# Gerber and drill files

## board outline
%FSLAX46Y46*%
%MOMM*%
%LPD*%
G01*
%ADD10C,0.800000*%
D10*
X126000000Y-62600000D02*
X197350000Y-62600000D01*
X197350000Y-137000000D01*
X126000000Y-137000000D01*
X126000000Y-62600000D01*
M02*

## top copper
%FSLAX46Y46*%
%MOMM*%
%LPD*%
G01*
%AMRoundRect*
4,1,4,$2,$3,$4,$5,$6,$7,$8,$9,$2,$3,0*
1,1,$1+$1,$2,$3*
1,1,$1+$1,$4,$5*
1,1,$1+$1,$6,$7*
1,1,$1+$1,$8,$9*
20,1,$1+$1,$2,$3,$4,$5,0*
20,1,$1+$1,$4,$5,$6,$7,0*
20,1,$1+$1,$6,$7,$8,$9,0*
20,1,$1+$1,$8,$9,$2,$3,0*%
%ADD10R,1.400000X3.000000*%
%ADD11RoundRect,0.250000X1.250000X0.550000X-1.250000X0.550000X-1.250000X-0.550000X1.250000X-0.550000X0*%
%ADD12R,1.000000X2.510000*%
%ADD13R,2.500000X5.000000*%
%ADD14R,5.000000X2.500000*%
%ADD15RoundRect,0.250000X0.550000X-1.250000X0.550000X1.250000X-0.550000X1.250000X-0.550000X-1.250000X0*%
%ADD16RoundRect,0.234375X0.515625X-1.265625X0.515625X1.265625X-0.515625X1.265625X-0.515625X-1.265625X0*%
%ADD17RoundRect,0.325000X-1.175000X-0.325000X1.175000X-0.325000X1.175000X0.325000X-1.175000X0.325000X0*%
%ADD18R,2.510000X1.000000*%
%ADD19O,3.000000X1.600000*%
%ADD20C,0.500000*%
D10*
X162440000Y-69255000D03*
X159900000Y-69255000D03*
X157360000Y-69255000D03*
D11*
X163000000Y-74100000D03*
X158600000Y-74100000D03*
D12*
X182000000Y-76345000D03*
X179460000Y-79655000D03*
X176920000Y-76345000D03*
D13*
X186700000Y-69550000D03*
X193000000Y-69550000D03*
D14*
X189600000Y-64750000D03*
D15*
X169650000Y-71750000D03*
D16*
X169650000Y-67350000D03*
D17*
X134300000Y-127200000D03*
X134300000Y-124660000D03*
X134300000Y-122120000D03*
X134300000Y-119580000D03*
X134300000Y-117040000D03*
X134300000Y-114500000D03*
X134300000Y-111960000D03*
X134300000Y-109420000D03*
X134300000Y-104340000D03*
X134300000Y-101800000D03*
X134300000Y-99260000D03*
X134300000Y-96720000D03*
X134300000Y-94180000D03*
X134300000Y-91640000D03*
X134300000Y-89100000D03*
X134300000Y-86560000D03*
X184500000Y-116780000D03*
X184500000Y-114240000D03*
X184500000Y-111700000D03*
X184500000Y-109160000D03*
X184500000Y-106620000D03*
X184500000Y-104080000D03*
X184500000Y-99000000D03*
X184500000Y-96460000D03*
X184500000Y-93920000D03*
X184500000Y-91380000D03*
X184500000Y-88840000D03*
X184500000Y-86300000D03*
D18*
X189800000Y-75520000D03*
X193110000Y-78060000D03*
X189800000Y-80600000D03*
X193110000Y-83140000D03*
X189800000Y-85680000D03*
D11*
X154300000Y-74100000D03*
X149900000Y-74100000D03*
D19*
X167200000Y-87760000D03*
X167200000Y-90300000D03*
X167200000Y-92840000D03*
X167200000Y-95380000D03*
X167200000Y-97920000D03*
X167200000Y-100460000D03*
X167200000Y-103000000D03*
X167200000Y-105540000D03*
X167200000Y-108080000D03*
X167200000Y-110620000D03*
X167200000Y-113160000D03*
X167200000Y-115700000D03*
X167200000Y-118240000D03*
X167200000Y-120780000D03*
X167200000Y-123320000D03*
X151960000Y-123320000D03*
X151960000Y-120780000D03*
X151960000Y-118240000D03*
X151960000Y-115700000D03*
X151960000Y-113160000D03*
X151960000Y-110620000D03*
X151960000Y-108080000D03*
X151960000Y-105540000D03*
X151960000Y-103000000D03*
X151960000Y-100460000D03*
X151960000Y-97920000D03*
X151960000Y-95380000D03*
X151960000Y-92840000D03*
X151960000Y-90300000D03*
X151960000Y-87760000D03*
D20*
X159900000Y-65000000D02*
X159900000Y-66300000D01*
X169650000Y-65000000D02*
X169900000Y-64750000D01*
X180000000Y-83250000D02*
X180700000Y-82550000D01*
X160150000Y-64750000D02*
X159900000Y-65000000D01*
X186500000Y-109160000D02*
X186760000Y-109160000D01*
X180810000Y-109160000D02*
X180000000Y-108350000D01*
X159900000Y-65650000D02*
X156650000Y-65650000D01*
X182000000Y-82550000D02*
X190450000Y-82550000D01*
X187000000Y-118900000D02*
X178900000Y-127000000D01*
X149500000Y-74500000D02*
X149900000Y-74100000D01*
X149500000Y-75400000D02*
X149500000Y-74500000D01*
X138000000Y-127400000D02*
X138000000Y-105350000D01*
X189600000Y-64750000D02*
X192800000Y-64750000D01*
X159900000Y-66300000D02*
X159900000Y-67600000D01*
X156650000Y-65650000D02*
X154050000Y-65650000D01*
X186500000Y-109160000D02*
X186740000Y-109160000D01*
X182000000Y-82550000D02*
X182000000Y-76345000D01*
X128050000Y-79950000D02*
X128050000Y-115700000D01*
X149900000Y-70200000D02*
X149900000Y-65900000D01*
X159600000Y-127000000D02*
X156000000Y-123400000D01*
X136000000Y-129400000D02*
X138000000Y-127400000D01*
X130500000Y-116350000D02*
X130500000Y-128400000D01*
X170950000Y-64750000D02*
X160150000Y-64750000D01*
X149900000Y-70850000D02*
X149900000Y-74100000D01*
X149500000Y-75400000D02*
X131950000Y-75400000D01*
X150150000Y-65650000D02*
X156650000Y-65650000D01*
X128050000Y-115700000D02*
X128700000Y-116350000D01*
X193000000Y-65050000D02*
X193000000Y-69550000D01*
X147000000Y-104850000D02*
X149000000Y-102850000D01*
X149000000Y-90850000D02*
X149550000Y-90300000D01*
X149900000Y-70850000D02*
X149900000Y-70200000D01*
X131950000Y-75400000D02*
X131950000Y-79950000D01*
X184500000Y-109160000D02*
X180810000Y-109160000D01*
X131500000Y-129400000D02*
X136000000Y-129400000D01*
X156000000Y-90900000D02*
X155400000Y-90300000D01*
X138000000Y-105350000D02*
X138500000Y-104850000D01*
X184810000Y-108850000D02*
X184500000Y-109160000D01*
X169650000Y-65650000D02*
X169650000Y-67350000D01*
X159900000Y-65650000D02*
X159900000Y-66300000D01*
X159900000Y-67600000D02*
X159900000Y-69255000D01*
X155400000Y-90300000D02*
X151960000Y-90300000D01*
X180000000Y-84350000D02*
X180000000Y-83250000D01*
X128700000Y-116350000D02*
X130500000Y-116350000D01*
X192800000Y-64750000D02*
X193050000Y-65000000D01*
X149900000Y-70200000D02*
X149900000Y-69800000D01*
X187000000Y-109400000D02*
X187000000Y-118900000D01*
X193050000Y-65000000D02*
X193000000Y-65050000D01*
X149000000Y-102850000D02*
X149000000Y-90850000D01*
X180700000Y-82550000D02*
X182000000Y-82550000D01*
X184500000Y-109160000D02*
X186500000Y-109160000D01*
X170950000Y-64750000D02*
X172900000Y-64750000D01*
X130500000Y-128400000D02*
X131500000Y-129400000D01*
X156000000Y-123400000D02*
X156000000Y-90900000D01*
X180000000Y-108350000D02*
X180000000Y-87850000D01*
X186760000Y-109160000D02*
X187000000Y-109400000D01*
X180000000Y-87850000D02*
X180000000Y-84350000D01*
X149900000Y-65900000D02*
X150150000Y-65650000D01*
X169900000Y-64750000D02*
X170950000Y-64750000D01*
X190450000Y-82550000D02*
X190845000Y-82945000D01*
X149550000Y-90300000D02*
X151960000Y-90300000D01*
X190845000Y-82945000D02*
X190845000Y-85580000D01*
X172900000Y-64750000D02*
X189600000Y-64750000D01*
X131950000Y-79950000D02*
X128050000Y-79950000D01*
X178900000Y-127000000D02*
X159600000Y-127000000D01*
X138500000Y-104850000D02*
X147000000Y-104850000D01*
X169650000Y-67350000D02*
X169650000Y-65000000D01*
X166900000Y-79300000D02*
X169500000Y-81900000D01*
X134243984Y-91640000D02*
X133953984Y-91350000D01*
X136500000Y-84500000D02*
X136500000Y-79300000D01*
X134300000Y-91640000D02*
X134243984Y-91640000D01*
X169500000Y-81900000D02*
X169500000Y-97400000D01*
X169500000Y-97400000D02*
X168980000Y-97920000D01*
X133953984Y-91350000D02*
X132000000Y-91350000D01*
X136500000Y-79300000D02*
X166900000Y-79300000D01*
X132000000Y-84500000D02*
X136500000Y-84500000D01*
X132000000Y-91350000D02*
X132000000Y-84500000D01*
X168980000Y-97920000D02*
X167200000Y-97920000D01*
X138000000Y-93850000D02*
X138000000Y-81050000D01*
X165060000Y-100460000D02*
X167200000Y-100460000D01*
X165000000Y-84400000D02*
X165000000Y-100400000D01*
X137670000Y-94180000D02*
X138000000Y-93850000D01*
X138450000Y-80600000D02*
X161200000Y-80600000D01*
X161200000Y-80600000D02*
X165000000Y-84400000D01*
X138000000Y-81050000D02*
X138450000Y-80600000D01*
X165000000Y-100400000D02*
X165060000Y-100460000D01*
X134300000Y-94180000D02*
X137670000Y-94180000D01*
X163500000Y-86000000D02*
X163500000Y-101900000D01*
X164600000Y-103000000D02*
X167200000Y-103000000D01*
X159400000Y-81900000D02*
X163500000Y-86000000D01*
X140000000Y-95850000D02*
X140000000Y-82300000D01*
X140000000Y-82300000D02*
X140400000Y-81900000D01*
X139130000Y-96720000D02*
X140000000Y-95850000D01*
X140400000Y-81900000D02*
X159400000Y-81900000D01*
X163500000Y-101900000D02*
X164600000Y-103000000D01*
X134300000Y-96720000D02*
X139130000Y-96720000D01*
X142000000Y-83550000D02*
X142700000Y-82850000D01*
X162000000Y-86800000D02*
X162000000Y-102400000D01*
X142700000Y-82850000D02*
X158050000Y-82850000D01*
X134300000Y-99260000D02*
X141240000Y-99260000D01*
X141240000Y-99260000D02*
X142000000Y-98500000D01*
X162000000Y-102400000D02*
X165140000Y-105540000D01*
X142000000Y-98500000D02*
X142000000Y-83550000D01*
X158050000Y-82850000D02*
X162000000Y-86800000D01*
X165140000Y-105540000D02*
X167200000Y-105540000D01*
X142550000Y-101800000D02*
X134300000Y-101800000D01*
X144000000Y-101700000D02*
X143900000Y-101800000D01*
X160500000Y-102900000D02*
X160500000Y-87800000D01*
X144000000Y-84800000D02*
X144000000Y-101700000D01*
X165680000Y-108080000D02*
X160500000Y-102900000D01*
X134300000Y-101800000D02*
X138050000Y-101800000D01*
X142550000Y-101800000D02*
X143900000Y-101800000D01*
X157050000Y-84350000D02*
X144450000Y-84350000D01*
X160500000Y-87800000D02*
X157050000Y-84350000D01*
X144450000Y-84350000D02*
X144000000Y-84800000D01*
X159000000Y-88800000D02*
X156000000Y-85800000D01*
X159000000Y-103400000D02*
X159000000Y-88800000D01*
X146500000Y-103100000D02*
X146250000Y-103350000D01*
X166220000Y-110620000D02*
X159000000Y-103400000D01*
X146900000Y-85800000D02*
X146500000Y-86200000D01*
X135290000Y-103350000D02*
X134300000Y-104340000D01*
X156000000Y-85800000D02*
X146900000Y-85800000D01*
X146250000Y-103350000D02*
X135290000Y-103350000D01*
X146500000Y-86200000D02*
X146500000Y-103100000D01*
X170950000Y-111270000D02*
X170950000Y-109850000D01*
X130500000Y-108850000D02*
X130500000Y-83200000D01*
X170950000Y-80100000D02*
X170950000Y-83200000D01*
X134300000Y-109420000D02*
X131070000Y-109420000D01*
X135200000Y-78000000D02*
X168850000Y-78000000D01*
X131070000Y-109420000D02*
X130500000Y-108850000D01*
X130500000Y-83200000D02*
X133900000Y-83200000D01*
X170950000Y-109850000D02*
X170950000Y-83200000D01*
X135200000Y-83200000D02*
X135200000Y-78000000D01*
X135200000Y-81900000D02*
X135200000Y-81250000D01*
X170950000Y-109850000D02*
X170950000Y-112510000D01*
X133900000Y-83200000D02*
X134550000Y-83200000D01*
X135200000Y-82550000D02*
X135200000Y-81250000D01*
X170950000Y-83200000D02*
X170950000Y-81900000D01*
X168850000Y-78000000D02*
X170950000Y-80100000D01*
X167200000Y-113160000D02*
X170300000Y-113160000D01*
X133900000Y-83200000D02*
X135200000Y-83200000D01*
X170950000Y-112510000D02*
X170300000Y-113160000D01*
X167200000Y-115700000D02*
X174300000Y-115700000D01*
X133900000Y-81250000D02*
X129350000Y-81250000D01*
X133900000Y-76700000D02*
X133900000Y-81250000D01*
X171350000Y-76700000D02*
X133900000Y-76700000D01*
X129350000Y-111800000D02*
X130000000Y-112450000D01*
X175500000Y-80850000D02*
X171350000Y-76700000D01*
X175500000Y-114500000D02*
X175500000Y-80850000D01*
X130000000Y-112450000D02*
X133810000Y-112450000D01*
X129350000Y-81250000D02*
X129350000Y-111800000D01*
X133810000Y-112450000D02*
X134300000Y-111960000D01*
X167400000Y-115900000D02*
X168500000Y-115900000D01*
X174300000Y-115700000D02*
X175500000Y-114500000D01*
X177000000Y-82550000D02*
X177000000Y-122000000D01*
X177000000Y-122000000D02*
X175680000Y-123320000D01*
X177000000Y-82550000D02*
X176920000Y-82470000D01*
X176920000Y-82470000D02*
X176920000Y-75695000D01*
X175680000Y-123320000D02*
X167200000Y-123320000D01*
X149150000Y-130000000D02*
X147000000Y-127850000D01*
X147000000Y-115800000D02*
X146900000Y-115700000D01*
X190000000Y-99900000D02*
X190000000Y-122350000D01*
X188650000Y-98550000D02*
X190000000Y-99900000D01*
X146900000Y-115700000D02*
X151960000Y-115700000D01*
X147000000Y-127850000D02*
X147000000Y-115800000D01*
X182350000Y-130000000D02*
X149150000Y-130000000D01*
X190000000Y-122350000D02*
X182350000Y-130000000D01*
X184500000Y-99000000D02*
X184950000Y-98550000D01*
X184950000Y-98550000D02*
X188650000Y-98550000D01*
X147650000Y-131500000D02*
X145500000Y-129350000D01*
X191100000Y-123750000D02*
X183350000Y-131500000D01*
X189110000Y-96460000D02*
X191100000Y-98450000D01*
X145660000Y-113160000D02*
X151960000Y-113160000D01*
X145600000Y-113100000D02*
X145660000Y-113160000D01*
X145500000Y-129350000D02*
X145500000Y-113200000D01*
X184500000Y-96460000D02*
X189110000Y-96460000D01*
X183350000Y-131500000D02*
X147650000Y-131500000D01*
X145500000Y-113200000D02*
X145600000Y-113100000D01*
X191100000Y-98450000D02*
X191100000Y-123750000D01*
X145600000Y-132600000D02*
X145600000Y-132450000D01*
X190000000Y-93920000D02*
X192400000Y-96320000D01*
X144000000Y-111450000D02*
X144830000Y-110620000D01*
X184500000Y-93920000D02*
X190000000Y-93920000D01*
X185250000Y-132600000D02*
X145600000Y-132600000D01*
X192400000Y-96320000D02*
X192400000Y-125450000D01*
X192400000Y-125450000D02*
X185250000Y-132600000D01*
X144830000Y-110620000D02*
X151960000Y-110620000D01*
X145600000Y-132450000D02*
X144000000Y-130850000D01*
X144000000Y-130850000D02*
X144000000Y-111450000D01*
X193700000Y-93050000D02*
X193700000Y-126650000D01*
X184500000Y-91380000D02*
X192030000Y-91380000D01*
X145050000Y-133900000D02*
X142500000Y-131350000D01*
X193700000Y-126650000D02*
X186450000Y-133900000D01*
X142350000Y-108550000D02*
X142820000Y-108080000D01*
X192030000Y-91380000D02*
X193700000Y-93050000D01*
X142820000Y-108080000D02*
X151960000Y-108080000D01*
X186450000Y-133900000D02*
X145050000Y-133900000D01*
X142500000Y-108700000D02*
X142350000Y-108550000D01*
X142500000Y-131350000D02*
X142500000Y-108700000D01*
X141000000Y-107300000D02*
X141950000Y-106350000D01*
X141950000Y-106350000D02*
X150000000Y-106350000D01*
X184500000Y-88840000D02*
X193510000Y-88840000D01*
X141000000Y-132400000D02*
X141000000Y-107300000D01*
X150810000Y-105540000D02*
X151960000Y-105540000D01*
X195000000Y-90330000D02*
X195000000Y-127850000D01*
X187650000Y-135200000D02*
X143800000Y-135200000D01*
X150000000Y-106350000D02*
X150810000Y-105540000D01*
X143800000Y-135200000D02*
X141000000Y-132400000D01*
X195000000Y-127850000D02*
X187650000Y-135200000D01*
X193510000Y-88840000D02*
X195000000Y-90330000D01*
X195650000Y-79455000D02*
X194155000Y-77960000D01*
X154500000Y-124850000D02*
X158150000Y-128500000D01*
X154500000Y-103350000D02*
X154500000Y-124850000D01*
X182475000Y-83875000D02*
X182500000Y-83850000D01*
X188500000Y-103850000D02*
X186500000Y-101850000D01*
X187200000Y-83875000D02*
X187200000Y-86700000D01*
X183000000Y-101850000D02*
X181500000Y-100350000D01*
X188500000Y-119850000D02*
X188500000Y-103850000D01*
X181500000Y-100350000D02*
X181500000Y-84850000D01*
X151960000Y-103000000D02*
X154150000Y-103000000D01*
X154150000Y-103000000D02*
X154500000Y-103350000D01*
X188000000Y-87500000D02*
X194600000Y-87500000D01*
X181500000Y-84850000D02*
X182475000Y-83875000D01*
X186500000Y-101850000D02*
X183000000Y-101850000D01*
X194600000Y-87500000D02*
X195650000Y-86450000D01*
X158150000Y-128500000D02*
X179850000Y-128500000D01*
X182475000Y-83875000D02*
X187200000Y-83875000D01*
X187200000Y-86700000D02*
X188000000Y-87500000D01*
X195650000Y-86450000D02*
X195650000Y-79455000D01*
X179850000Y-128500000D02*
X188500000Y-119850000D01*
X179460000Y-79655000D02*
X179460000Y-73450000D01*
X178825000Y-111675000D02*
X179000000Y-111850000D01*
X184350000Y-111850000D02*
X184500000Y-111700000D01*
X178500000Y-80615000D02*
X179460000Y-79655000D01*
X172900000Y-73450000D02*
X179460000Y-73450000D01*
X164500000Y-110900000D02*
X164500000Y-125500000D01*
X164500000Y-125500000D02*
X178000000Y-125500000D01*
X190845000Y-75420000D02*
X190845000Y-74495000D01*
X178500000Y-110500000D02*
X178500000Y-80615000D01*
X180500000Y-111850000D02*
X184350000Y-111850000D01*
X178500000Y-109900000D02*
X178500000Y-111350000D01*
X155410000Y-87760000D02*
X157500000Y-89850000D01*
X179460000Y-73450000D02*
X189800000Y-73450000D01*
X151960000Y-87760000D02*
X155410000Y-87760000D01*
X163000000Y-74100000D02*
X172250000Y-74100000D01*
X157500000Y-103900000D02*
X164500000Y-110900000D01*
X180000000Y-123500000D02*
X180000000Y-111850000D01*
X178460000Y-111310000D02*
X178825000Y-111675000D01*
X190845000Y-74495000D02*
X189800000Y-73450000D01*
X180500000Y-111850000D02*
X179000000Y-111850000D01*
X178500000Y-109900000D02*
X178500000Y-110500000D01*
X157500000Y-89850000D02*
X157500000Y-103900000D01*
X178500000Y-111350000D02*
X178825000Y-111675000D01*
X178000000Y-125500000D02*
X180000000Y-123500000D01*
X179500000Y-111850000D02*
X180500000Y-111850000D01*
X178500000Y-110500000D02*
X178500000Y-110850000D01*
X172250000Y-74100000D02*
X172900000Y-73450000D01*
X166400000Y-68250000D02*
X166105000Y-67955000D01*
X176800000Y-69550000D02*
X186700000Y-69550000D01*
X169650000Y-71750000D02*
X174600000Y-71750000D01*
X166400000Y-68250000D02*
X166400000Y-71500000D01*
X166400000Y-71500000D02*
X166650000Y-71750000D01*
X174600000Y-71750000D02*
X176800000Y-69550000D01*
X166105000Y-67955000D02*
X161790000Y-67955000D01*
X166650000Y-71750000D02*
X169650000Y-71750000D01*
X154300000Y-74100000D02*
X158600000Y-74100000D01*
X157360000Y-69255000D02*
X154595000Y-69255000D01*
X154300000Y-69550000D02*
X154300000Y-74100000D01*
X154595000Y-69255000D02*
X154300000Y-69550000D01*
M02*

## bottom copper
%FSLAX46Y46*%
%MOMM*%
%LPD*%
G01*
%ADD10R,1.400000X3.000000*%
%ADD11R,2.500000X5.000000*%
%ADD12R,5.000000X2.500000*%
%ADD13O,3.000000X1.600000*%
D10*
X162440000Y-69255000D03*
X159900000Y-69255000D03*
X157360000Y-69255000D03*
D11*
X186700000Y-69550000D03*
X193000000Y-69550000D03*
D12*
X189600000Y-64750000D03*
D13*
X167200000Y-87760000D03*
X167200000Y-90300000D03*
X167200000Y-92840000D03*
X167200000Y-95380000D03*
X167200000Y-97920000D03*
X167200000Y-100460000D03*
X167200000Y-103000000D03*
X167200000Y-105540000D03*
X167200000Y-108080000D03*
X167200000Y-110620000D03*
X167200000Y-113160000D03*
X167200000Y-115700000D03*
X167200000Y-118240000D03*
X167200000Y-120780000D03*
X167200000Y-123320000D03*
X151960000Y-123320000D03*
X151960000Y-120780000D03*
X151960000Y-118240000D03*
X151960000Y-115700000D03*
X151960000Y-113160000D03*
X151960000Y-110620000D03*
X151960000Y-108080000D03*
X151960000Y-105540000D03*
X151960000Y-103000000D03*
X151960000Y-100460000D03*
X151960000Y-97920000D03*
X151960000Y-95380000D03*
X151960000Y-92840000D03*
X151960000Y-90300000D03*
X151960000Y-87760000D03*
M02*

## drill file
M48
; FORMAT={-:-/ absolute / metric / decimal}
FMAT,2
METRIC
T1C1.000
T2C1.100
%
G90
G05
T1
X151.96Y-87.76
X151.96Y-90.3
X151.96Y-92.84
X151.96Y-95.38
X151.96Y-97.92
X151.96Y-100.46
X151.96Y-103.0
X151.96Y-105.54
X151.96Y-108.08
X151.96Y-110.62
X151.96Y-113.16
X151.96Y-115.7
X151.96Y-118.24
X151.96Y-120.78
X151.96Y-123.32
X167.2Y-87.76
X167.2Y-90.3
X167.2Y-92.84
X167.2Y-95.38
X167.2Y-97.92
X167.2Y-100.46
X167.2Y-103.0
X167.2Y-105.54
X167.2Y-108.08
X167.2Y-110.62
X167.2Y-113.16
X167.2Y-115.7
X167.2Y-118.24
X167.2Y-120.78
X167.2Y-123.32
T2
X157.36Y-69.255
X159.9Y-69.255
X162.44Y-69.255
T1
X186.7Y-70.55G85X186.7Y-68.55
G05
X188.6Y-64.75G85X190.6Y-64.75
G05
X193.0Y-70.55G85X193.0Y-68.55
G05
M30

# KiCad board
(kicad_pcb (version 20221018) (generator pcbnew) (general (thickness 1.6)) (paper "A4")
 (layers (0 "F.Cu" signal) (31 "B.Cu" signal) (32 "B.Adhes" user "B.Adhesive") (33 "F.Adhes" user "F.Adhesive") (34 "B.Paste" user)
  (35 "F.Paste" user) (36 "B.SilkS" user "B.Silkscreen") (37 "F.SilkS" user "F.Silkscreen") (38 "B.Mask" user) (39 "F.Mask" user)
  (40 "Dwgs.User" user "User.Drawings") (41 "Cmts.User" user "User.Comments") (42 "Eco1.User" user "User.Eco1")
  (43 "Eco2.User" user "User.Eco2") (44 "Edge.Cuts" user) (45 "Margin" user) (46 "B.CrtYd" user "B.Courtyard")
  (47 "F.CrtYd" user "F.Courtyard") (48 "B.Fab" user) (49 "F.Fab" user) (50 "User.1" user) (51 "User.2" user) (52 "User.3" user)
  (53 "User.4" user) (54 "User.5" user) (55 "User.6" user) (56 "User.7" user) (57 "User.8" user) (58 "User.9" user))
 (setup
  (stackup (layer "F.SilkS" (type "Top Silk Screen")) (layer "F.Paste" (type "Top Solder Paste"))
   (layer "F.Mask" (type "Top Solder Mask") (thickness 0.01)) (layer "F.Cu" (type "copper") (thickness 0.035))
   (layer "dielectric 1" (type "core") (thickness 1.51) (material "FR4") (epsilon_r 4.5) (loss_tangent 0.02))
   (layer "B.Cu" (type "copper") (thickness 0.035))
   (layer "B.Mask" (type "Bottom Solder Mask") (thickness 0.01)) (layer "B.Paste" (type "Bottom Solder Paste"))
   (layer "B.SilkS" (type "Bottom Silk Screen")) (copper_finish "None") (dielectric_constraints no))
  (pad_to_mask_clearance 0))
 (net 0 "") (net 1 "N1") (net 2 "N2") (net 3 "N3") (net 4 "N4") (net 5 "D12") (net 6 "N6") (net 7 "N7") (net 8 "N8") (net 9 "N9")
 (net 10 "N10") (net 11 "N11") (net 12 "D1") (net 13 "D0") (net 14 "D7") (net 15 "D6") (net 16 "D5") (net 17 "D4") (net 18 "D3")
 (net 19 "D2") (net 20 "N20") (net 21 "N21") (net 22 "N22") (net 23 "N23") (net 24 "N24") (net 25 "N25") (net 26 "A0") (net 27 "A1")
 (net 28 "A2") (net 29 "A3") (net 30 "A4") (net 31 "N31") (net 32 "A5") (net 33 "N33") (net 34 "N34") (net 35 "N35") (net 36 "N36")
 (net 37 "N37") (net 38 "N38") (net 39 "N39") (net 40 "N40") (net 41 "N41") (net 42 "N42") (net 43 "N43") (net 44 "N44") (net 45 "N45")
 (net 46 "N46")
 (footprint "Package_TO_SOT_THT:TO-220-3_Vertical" (layer "F.Cu") (at 162.44 69.255 180)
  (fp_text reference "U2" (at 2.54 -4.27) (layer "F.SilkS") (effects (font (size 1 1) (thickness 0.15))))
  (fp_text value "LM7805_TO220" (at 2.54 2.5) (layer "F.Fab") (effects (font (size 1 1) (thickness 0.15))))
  (pad "1" thru_hole rect (at 0 0 180) (size 1.4 3) (drill 1.1) (layers "*.Cu" "*.Mask") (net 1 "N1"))
  (pad "2" thru_hole rect (at 2.54 0 180) (size 1.4 3) (drill 1.1) (layers "*.Cu" "*.Mask") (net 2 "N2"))
  (pad "3" thru_hole rect (at 5.08 0 180) (size 1.4 3) (drill 1.1) (layers "*.Cu" "*.Mask") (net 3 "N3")))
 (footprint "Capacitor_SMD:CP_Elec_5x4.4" (layer "F.Cu") (at 160.8 74.1 180)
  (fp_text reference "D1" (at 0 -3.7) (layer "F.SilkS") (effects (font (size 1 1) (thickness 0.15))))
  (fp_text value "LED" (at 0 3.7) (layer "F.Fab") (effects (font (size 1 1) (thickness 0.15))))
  (pad "1" smd roundrect (at -2.2 0 180) (size 3 1.6) (layers "F.Cu" "F.Paste" "F.Mask") (roundrect_rratio 0.15625) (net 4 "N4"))
  (pad "2" smd roundrect (at 2.2 0 180) (size 3 1.6) (layers "F.Cu" "F.Paste" "F.Mask") (roundrect_rratio 0.15625) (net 3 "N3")))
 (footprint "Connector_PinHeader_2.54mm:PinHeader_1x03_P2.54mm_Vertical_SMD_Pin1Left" (layer "F.Cu") (at 179.46 78 -90)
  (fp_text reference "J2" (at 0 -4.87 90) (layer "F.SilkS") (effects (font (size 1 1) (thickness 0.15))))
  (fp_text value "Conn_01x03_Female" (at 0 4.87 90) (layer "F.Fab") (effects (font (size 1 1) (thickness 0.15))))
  (pad "1" smd rect (at -1.655 -2.54 270) (size 2.51 1) (layers "F.Cu" "F.Paste" "F.Mask") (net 2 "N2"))
  (pad "2" smd rect (at 1.655 0 270) (size 2.51 1) (layers "F.Cu" "F.Paste" "F.Mask") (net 4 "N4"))
  (pad "3" smd rect (at -1.655 2.54 270) (size 2.51 1) (layers "F.Cu" "F.Paste" "F.Mask") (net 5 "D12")))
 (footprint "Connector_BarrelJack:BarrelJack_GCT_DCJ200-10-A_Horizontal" (layer "F.Cu") (at 186.7 69.55 90)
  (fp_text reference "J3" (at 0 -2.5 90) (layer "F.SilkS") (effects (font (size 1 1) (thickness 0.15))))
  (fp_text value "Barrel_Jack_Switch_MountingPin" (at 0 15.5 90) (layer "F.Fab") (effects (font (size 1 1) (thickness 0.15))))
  (pad "1" thru_hole rect (at 0 0 90) (size 5 2.5) (drill oval 3 1) (layers "*.Cu" "*.Mask") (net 1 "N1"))
  (pad "2" thru_hole rect (at 0 6.3 90) (size 5 2.5) (drill oval 3 1) (layers "*.Cu" "*.Mask") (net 2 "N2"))
  (pad "3" thru_hole rect (at 4.8 2.9 90) (size 2.5 5) (drill oval 1 3) (layers "*.Cu" "*.Mask") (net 2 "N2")))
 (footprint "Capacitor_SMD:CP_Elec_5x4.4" (layer "F.Cu") (at 169.65 69.55 90)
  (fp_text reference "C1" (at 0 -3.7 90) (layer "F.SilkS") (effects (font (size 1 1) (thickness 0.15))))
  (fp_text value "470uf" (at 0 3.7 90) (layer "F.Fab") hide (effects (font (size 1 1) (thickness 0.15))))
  (pad "1" smd roundrect (at -2.2 0 90) (size 3 1.6) (layers "F.Cu" "F.Paste" "F.Mask") (roundrect_rratio 0.15625) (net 1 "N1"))
  (pad "2" smd roundrect (at 2.2 0 90) (size 3 1.5) (layers "F.Cu" "F.Paste" "F.Mask") (roundrect_rratio 0.15625) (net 2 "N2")))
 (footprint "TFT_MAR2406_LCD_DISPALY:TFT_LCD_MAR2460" (layer "F.Cu") (at 134.3 127.2)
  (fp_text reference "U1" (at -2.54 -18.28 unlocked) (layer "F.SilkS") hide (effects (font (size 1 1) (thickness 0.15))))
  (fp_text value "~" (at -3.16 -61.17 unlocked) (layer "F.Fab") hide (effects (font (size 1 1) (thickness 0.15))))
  (pad "1" smd roundrect (at 0 0) (size 3 1.3) (layers "F.Cu" "F.Paste" "F.Mask") (roundrect_rratio 0.25) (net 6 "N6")
   (thermal_bridge_angle 45))
  (pad "2" smd roundrect (at 0 -2.54) (size 3 1.3) (layers "F.Cu" "F.Paste" "F.Mask") (roundrect_rratio 0.25) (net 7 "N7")
   (thermal_bridge_angle 45))
  (pad "3" smd roundrect (at 0 -5.08) (size 3 1.3) (layers "F.Cu" "F.Paste" "F.Mask") (roundrect_rratio 0.25) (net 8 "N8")
   (thermal_bridge_angle 45))
  (pad "4" smd roundrect (at 0 -7.62) (size 3 1.3) (layers "F.Cu" "F.Paste" "F.Mask") (roundrect_rratio 0.25) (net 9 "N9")
   (thermal_bridge_angle 45))
  (pad "5" smd roundrect (at 0 -10.16) (size 3 1.3) (layers "F.Cu" "F.Paste" "F.Mask") (roundrect_rratio 0.25) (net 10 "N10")
   (thermal_bridge_angle 45))
  (pad "6" smd roundrect (at 0 -12.7) (size 3 1.3) (layers "F.Cu" "F.Paste" "F.Mask") (roundrect_rratio 0.25) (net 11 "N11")
   (thermal_bridge_angle 45))
  (pad "7" smd roundrect (at 0 -15.24) (size 3 1.3) (layers "F.Cu" "F.Paste" "F.Mask") (roundrect_rratio 0.25) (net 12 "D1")
   (thermal_bridge_angle 45))
  (pad "8" smd roundrect (at 0 -17.78) (size 3 1.3) (layers "F.Cu" "F.Paste" "F.Mask") (roundrect_rratio 0.25) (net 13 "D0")
   (thermal_bridge_angle 45))
  (pad "9" smd roundrect (at 0 -22.86) (size 3 1.3) (layers "F.Cu" "F.Paste" "F.Mask") (roundrect_rratio 0.25) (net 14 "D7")
   (thermal_bridge_angle 45))
  (pad "10" smd roundrect (at 0 -25.4) (size 3 1.3) (layers "F.Cu" "F.Paste" "F.Mask") (roundrect_rratio 0.25) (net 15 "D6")
   (thermal_bridge_angle 45))
  (pad "11" smd roundrect (at 0 -27.94) (size 3 1.3) (layers "F.Cu" "F.Paste" "F.Mask") (roundrect_rratio 0.25) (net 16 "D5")
   (thermal_bridge_angle 45))
  (pad "12" smd roundrect (at 0 -30.48) (size 3 1.3) (layers "F.Cu" "F.Paste" "F.Mask") (roundrect_rratio 0.25) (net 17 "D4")
   (thermal_bridge_angle 45))
  (pad "13" smd roundrect (at 0 -33.02) (size 3 1.3) (layers "F.Cu" "F.Paste" "F.Mask") (roundrect_rratio 0.25) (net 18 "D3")
   (thermal_bridge_angle 45))
  (pad "14" smd roundrect (at 0 -35.56) (size 3 1.3) (layers "F.Cu" "F.Paste" "F.Mask") (roundrect_rratio 0.25) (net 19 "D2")
   (thermal_bridge_angle 45))
  (pad "15" smd roundrect (at 0 -38.1) (size 3 1.3) (layers "F.Cu" "F.Paste" "F.Mask") (roundrect_rratio 0.25) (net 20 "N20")
   (thermal_bridge_angle 45))
  (pad "16" smd roundrect (at 0 -40.64) (size 3 1.3) (layers "F.Cu" "F.Paste" "F.Mask") (roundrect_rratio 0.25) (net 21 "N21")
   (thermal_bridge_angle 45))
  (pad "17" smd roundrect (at 50.2 -10.42) (size 3 1.3) (layers "F.Cu" "F.Paste" "F.Mask") (roundrect_rratio 0.25) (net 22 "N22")
   (thermal_bridge_angle 45))
  (pad "18" smd roundrect (at 50.2 -12.96) (size 3 1.3) (layers "F.Cu" "F.Paste" "F.Mask") (roundrect_rratio 0.25) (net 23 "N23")
   (thermal_bridge_angle 45))
  (pad "19" smd roundrect (at 50.2 -15.5) (size 3 1.3) (layers "F.Cu" "F.Paste" "F.Mask") (roundrect_rratio 0.25) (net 4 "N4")
   (thermal_bridge_angle 45))
  (pad "20" smd roundrect (at 50.2 -18.04) (size 3 1.3) (layers "F.Cu" "F.Paste" "F.Mask") (roundrect_rratio 0.25) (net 2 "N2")
   (thermal_bridge_angle 45))
  (pad "21" smd roundrect (at 50.2 -20.58) (size 3 1.3) (layers "F.Cu" "F.Paste" "F.Mask") (roundrect_rratio 0.25) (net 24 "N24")
   (thermal_bridge_angle 45))
  (pad "22" smd roundrect (at 50.2 -23.12) (size 3 1.3) (layers "F.Cu" "F.Paste" "F.Mask") (roundrect_rratio 0.25) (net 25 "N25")
   (thermal_bridge_angle 45))
  (pad "23" smd roundrect (at 50.2 -28.2) (size 3 1.3) (layers "F.Cu" "F.Paste" "F.Mask") (roundrect_rratio 0.25) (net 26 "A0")
   (thermal_bridge_angle 45))
  (pad "24" smd roundrect (at 50.2 -30.74) (size 3 1.3) (layers "F.Cu" "F.Paste" "F.Mask") (roundrect_rratio 0.25) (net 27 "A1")
   (thermal_bridge_angle 45))
  (pad "25" smd roundrect (at 50.2 -33.28) (size 3 1.3) (layers "F.Cu" "F.Paste" "F.Mask") (roundrect_rratio 0.25) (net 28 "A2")
   (thermal_bridge_angle 45))
  (pad "26" smd roundrect (at 50.2 -35.82) (size 3 1.3) (layers "F.Cu" "F.Paste" "F.Mask") (roundrect_rratio 0.25) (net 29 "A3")
   (thermal_bridge_angle 45))
  (pad "27" smd roundrect (at 50.2 -38.36) (size 3 1.3) (layers "F.Cu" "F.Paste" "F.Mask") (roundrect_rratio 0.25) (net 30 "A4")
   (thermal_bridge_angle 45))
  (pad "28" smd roundrect (at 50.2 -40.9) (size 3 1.3) (layers "F.Cu" "F.Paste" "F.Mask") (roundrect_rratio 0.25) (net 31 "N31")
   (thermal_bridge_angle 45)))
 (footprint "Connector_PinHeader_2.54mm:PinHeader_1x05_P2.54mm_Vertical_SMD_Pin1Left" (layer "F.Cu") (at 191.455 80.6)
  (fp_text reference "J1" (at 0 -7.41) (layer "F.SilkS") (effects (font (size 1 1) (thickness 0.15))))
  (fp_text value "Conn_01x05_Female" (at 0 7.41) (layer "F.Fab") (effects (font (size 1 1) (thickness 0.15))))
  (pad "1" smd rect (at -1.655 -5.08) (size 2.51 1) (layers "F.Cu" "F.Paste" "F.Mask") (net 4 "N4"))
  (pad "2" smd rect (at 1.655 -2.54) (size 2.51 1) (layers "F.Cu" "F.Paste" "F.Mask") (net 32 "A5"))
  (pad "3" smd rect (at -1.655 0) (size 2.51 1) (layers "F.Cu" "F.Paste" "F.Mask") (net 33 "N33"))
  (pad "4" smd rect (at 1.655 2.54) (size 2.51 1) (layers "F.Cu" "F.Paste" "F.Mask") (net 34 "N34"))
  (pad "5" smd rect (at -1.655 5.08) (size 2.51 1) (layers "F.Cu" "F.Paste" "F.Mask") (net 2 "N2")))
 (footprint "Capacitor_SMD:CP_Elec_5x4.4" (layer "F.Cu") (at 152.1 74.1 180)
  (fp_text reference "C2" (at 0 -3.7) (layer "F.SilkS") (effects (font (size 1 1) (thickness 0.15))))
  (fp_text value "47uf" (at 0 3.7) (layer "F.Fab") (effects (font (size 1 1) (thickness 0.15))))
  (pad "1" smd roundrect (at -2.2 0 180) (size 3 1.6) (layers "F.Cu" "F.Paste" "F.Mask") (roundrect_rratio 0.15625) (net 3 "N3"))
  (pad "2" smd roundrect (at 2.2 0 180) (size 3 1.6) (layers "F.Cu" "F.Paste" "F.Mask") (roundrect_rratio 0.15625) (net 2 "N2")))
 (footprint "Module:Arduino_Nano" (layer "B.Cu") (at 167.2 87.76 180)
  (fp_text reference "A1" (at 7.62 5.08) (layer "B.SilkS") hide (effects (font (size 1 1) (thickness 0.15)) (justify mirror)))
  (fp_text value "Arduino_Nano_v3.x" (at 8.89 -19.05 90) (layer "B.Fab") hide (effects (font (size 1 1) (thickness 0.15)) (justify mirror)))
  (pad "1" thru_hole oval (at 0 0 180) (size 3 1.6) (drill 1) (layers "*.Cu" "*.Mask") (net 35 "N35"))
  (pad "2" thru_hole oval (at 0 -2.54 180) (size 3 1.6) (drill 1) (layers "*.Cu" "*.Mask") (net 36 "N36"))
  (pad "3" thru_hole oval (at 0 -5.08 180) (size 3 1.6) (drill 1) (layers "*.Cu" "*.Mask") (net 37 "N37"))
  (pad "4" thru_hole oval (at 0 -7.62 180) (size 3 1.6) (drill 1) (layers "*.Cu" "*.Mask") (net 2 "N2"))
  (pad "5" thru_hole oval (at 0 -10.16 180) (size 3 1.6) (drill 1) (layers "*.Cu" "*.Mask") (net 19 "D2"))
  (pad "6" thru_hole oval (at 0 -12.7 180) (size 3 1.6) (drill 1) (layers "*.Cu" "*.Mask") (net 18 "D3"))
  (pad "7" thru_hole oval (at 0 -15.24 180) (size 3 1.6) (drill 1) (layers "*.Cu" "*.Mask") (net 17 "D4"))
  (pad "8" thru_hole oval (at 0 -17.78 180) (size 3 1.6) (drill 1) (layers "*.Cu" "*.Mask") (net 16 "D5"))
  (pad "9" thru_hole oval (at 0 -20.32 180) (size 3 1.6) (drill 1) (layers "*.Cu" "*.Mask") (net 15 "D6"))
  (pad "10" thru_hole oval (at 0 -22.86 180) (size 3 1.6) (drill 1) (layers "*.Cu" "*.Mask") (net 14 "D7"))
  (pad "11" thru_hole oval (at 0 -25.4 180) (size 3 1.6) (drill 1) (layers "*.Cu" "*.Mask") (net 13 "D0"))
  (pad "12" thru_hole oval (at 0 -27.94 180) (size 3 1.6) (drill 1) (layers "*.Cu" "*.Mask") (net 12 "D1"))
  (pad "13" thru_hole oval (at 0 -30.48 180) (size 3 1.6) (drill 1) (layers "*.Cu" "*.Mask") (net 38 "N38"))
  (pad "14" thru_hole oval (at 0 -33.02 180) (size 3 1.6) (drill 1) (layers "*.Cu" "*.Mask") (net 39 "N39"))
  (pad "15" thru_hole oval (at 0 -35.56 180) (size 3 1.6) (drill 1) (layers "*.Cu" "*.Mask") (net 5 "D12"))
  (pad "16" thru_hole oval (at 15.24 -35.56 180) (size 3 1.6) (drill 1) (layers "*.Cu" "*.Mask") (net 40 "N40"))
  (pad "17" thru_hole oval (at 15.24 -33.02 180) (size 3 1.6) (drill 1) (layers "*.Cu" "*.Mask") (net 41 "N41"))
  (pad "18" thru_hole oval (at 15.24 -30.48 180) (size 3 1.6) (drill 1) (layers "*.Cu" "*.Mask") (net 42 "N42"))
  (pad "19" thru_hole oval (at 15.24 -27.94 180) (size 3 1.6) (drill 1) (layers "*.Cu" "*.Mask") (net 26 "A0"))
  (pad "20" thru_hole oval (at 15.24 -25.4 180) (size 3 1.6) (drill 1) (layers "*.Cu" "*.Mask") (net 27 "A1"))
  (pad "21" thru_hole oval (at 15.24 -22.86 180) (size 3 1.6) (drill 1) (layers "*.Cu" "*.Mask") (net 28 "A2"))
  (pad "22" thru_hole oval (at 15.24 -20.32 180) (size 3 1.6) (drill 1) (layers "*.Cu" "*.Mask") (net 29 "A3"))
  (pad "23" thru_hole oval (at 15.24 -17.78 180) (size 3 1.6) (drill 1) (layers "*.Cu" "*.Mask") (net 30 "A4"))
  (pad "24" thru_hole oval (at 15.24 -15.24 180) (size 3 1.6) (drill 1) (layers "*.Cu" "*.Mask") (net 32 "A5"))
  (pad "25" thru_hole oval (at 15.24 -12.7 180) (size 3 1.6) (drill 1) (layers "*.Cu" "*.Mask") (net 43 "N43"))
  (pad "26" thru_hole oval (at 15.24 -10.16 180) (size 3 1.6) (drill 1) (layers "*.Cu" "*.Mask") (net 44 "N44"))
  (pad "27" thru_hole oval (at 15.24 -7.62 180) (size 3 1.6) (drill 1) (layers "*.Cu" "*.Mask") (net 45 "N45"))
  (pad "28" thru_hole oval (at 15.24 -5.08 180) (size 3 1.6) (drill 1) (layers "*.Cu" "*.Mask") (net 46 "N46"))
  (pad "29" thru_hole oval (at 15.24 -2.54 180) (size 3 1.6) (drill 1) (layers "*.Cu" "*.Mask") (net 2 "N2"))
  (pad "30" thru_hole oval (at 15.24 0 180) (size 3 1.6) (drill 1) (layers "*.Cu" "*.Mask") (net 4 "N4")))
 (gr_rect (start 126 62.6) (end 197.35 137) (stroke (width 0.8) (type default)) (fill none) (layer "Edge.Cuts"))
 (segment (start 159.9 65) (end 159.9 66.3) (width 0.5) (layer "F.Cu") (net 2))
 (segment (start 169.65 65) (end 169.9 64.75) (width 0.5) (layer "F.Cu") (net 2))
 (segment (start 180 83.25) (end 180.7 82.55) (width 0.5) (layer "F.Cu") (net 2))
 (segment (start 160.15 64.75) (end 159.9 65) (width 0.5) (layer "F.Cu") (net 2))
 (segment (start 186.5 109.16) (end 186.76 109.16) (width 0.5) (layer "F.Cu") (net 2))
 (segment (start 180.81 109.16) (end 180 108.35) (width 0.5) (layer "F.Cu") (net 2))
 (segment (start 159.9 65.65) (end 156.65 65.65) (width 0.5) (layer "F.Cu") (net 2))
 (segment (start 182 82.55) (end 190.45 82.55) (width 0.5) (layer "F.Cu") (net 2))
 (segment (start 187 118.9) (end 178.9 127) (width 0.5) (layer "F.Cu") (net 2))
 (segment (start 149.5 74.5) (end 149.9 74.1) (width 0.5) (layer "F.Cu") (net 2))
 (segment (start 149.5 75.4) (end 149.5 74.5) (width 0.5) (layer "F.Cu") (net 2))
 (segment (start 138 127.4) (end 138 105.35) (width 0.5) (layer "F.Cu") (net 2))
 (segment (start 189.6 64.75) (end 192.8 64.75) (width 0.5) (layer "F.Cu") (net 2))
 (segment (start 159.9 66.3) (end 159.9 67.6) (width 0.5) (layer "F.Cu") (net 2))
 (segment (start 156.65 65.65) (end 154.05 65.65) (width 0.5) (layer "F.Cu") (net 2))
 (segment (start 186.5 109.16) (end 186.74 109.16) (width 0.5) (layer "F.Cu") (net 2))
 (segment (start 182 82.55) (end 182 76.345) (width 0.5) (layer "F.Cu") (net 2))
 (segment (start 128.05 79.95) (end 128.05 115.7) (width 0.5) (layer "F.Cu") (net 2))
 (segment (start 149.9 70.2) (end 149.9 65.9) (width 0.5) (layer "F.Cu") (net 2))
 (segment (start 159.6 127) (end 156 123.4) (width 0.5) (layer "F.Cu") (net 2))
 (segment (start 136 129.4) (end 138 127.4) (width 0.5) (layer "F.Cu") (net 2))
 (segment (start 130.5 116.35) (end 130.5 128.4) (width 0.5) (layer "F.Cu") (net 2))
 (segment (start 170.95 64.75) (end 160.15 64.75) (width 0.5) (layer "F.Cu") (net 2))
 (segment (start 149.9 70.85) (end 149.9 74.1) (width 0.5) (layer "F.Cu") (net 2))
 (segment (start 149.5 75.4) (end 131.95 75.4) (width 0.5) (layer "F.Cu") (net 2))
 (segment (start 150.15 65.65) (end 156.65 65.65) (width 0.5) (layer "F.Cu") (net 2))
 (segment (start 128.05 115.7) (end 128.7 116.35) (width 0.5) (layer "F.Cu") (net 2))
 (segment (start 193 65.05) (end 193 69.55) (width 0.5) (layer "F.Cu") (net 2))
 (segment (start 147 104.85) (end 149 102.85) (width 0.5) (layer "F.Cu") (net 2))
 (segment (start 149 90.85) (end 149.55 90.3) (width 0.5) (layer "F.Cu") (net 2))
 (segment (start 149.9 70.85) (end 149.9 70.2) (width 0.5) (layer "F.Cu") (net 2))
 (segment (start 131.95 75.4) (end 131.95 79.95) (width 0.5) (layer "F.Cu") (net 2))
 (segment (start 184.5 109.16) (end 180.81 109.16) (width 0.5) (layer "F.Cu") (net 2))
 (segment (start 131.5 129.4) (end 136 129.4) (width 0.5) (layer "F.Cu") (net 2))
 (segment (start 156 90.9) (end 155.4 90.3) (width 0.5) (layer "F.Cu") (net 2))
 (segment (start 138 105.35) (end 138.5 104.85) (width 0.5) (layer "F.Cu") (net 2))
 (segment (start 184.81 108.85) (end 184.5 109.16) (width 0.5) (layer "F.Cu") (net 2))
 (segment (start 169.65 65.65) (end 169.65 67.35) (width 0.5) (layer "F.Cu") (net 2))
 (segment (start 159.9 65.65) (end 159.9 66.3) (width 0.5) (layer "F.Cu") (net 2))
 (segment (start 159.9 67.6) (end 159.9 69.255) (width 0.5) (layer "F.Cu") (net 2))
 (segment (start 155.4 90.3) (end 151.96 90.3) (width 0.5) (layer "F.Cu") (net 2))
 (segment (start 180 84.35) (end 180 83.25) (width 0.5) (layer "F.Cu") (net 2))
 (segment (start 128.7 116.35) (end 130.5 116.35) (width 0.5) (layer "F.Cu") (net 2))
 (segment (start 192.8 64.75) (end 193.05 65) (width 0.5) (layer "F.Cu") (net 2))
 (segment (start 149.9 70.2) (end 149.9 69.8) (width 0.5) (layer "F.Cu") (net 2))
 (segment (start 187 109.4) (end 187 118.9) (width 0.5) (layer "F.Cu") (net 2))
 (segment (start 193.05 65) (end 193 65.05) (width 0.5) (layer "F.Cu") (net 2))
 (segment (start 149 102.85) (end 149 90.85) (width 0.5) (layer "F.Cu") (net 2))
 (segment (start 180.7 82.55) (end 182 82.55) (width 0.5) (layer "F.Cu") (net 2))
 (segment (start 184.5 109.16) (end 186.5 109.16) (width 0.5) (layer "F.Cu") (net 2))
 (segment (start 170.95 64.75) (end 172.9 64.75) (width 0.5) (layer "F.Cu") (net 2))
 (segment (start 130.5 128.4) (end 131.5 129.4) (width 0.5) (layer "F.Cu") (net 2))
 (segment (start 156 123.4) (end 156 90.9) (width 0.5) (layer "F.Cu") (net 2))
 (segment (start 180 108.35) (end 180 87.85) (width 0.5) (layer "F.Cu") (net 2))
 (segment (start 186.76 109.16) (end 187 109.4) (width 0.5) (layer "F.Cu") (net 2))
 (segment (start 180 87.85) (end 180 84.35) (width 0.5) (layer "F.Cu") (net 2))
 (segment (start 149.9 65.9) (end 150.15 65.65) (width 0.5) (layer "F.Cu") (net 2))
 (segment (start 169.9 64.75) (end 170.95 64.75) (width 0.5) (layer "F.Cu") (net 2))
 (segment (start 190.45 82.55) (end 190.845 82.945) (width 0.5) (layer "F.Cu") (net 2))
 (segment (start 149.55 90.3) (end 151.96 90.3) (width 0.5) (layer "F.Cu") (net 2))
 (segment (start 190.845 82.945) (end 190.845 85.58) (width 0.5) (layer "F.Cu") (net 2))
 (segment (start 172.9 64.75) (end 189.6 64.75) (width 0.5) (layer "F.Cu") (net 2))
 (segment (start 131.95 79.95) (end 128.05 79.95) (width 0.5) (layer "F.Cu") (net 2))
 (segment (start 178.9 127) (end 159.6 127) (width 0.5) (layer "F.Cu") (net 2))
 (segment (start 138.5 104.85) (end 147 104.85) (width 0.5) (layer "F.Cu") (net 2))
 (segment (start 169.65 67.35) (end 169.65 65) (width 0.5) (layer "F.Cu") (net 2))
 (segment (start 166.9 79.3) (end 169.5 81.9) (width 0.5) (layer "F.Cu") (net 19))
 (segment (start 134.243984 91.64) (end 133.953984 91.35) (width 0.5) (layer "F.Cu") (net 19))
 (segment (start 136.5 84.5) (end 136.5 79.3) (width 0.5) (layer "F.Cu") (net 19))
 (segment (start 134.3 91.64) (end 134.243984 91.64) (width 0.5) (layer "F.Cu") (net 19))
 (segment (start 169.5 81.9) (end 169.5 97.4) (width 0.5) (layer "F.Cu") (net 19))
 (segment (start 169.5 97.4) (end 168.98 97.92) (width 0.5) (layer "F.Cu") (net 19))
 (segment (start 133.953984 91.35) (end 132 91.35) (width 0.5) (layer "F.Cu") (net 19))
 (segment (start 136.5 79.3) (end 166.9 79.3) (width 0.5) (layer "F.Cu") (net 19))
 (segment (start 132 84.5) (end 136.5 84.5) (width 0.5) (layer "F.Cu") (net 19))
 (segment (start 132 91.35) (end 132 84.5) (width 0.5) (layer "F.Cu") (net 19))
 (segment (start 168.98 97.92) (end 167.2 97.92) (width 0.5) (layer "F.Cu") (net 19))
 (segment (start 138 93.85) (end 138 81.05) (width 0.5) (layer "F.Cu") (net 18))
 (segment (start 165.06 100.46) (end 167.2 100.46) (width 0.5) (layer "F.Cu") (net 18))
 (segment (start 165 84.4) (end 165 100.4) (width 0.5) (layer "F.Cu") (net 18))
 (segment (start 137.67 94.18) (end 138 93.85) (width 0.5) (layer "F.Cu") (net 18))
 (segment (start 138.45 80.6) (end 161.2 80.6) (width 0.5) (layer "F.Cu") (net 18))
 (segment (start 161.2 80.6) (end 165 84.4) (width 0.5) (layer "F.Cu") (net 18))
 (segment (start 138 81.05) (end 138.45 80.6) (width 0.5) (layer "F.Cu") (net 18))
 (segment (start 165 100.4) (end 165.06 100.46) (width 0.5) (layer "F.Cu") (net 18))
 (segment (start 134.3 94.18) (end 137.67 94.18) (width 0.5) (layer "F.Cu") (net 18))
 (segment (start 163.5 86) (end 163.5 101.9) (width 0.5) (layer "F.Cu") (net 17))
 (segment (start 164.6 103) (end 167.2 103) (width 0.5) (layer "F.Cu") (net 17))
 (segment (start 159.4 81.9) (end 163.5 86) (width 0.5) (layer "F.Cu") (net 17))
 (segment (start 140 95.85) (end 140 82.3) (width 0.5) (layer "F.Cu") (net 17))
 (segment (start 140 82.3) (end 140.4 81.9) (width 0.5) (layer "F.Cu") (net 17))
 (segment (start 139.13 96.72) (end 140 95.85) (width 0.5) (layer "F.Cu") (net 17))
 (segment (start 140.4 81.9) (end 159.4 81.9) (width 0.5) (layer "F.Cu") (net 17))
 (segment (start 163.5 101.9) (end 164.6 103) (width 0.5) (layer "F.Cu") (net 17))
 (segment (start 134.3 96.72) (end 139.13 96.72) (width 0.5) (layer "F.Cu") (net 17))
 (segment (start 142 83.55) (end 142.7 82.85) (width 0.5) (layer "F.Cu") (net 16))
 (segment (start 162 86.8) (end 162 102.4) (width 0.5) (layer "F.Cu") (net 16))
 (segment (start 142.7 82.85) (end 158.05 82.85) (width 0.5) (layer "F.Cu") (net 16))
 (segment (start 134.3 99.26) (end 141.24 99.26) (width 0.5) (layer "F.Cu") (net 16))
 (segment (start 141.24 99.26) (end 142 98.5) (width 0.5) (layer "F.Cu") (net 16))
 (segment (start 162 102.4) (end 165.14 105.54) (width 0.5) (layer "F.Cu") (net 16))
 (segment (start 142 98.5) (end 142 83.55) (width 0.5) (layer "F.Cu") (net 16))
 (segment (start 158.05 82.85) (end 162 86.8) (width 0.5) (layer "F.Cu") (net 16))
 (segment (start 165.14 105.54) (end 167.2 105.54) (width 0.5) (layer "F.Cu") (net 16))
 (segment (start 142.55 101.8) (end 134.3 101.8) (width 0.5) (layer "F.Cu") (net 15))
 (segment (start 144 101.7) (end 143.9 101.8) (width 0.5) (layer "F.Cu") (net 15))
 (segment (start 160.5 102.9) (end 160.5 87.8) (width 0.5) (layer "F.Cu") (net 15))
 (segment (start 144 84.8) (end 144 101.7) (width 0.5) (layer "F.Cu") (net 15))
 (segment (start 165.68 108.08) (end 160.5 102.9) (width 0.5) (layer "F.Cu") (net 15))
 (segment (start 134.3 101.8) (end 138.05 101.8) (width 0.5) (layer "F.Cu") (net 15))
 (segment (start 142.55 101.8) (end 143.9 101.8) (width 0.5) (layer "F.Cu") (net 15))
 (segment (start 157.05 84.35) (end 144.45 84.35) (width 0.5) (layer "F.Cu") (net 15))
 (segment (start 160.5 87.8) (end 157.05 84.35) (width 0.5) (layer "F.Cu") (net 15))
 (segment (start 144.45 84.35) (end 144 84.8) (width 0.5) (layer "F.Cu") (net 15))
 (segment (start 159 88.8) (end 156 85.8) (width 0.5) (layer "F.Cu") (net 14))
 (segment (start 159 103.4) (end 159 88.8) (width 0.5) (layer "F.Cu") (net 14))
 (segment (start 146.5 103.1) (end 146.25 103.35) (width 0.5) (layer "F.Cu") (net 14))
 (segment (start 166.22 110.62) (end 159 103.4) (width 0.5) (layer "F.Cu") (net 14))
 (segment (start 146.9 85.8) (end 146.5 86.2) (width 0.5) (layer "F.Cu") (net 14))
 (segment (start 135.29 103.35) (end 134.3 104.34) (width 0.5) (layer "F.Cu") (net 14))
 (segment (start 156 85.8) (end 146.9 85.8) (width 0.5) (layer "F.Cu") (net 14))
 (segment (start 146.25 103.35) (end 135.29 103.35) (width 0.5) (layer "F.Cu") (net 14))
 (segment (start 146.5 86.2) (end 146.5 103.1) (width 0.5) (layer "F.Cu") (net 14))
 (segment (start 170.95 111.27) (end 170.95 109.85) (width 0.5) (layer "F.Cu") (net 13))
 (segment (start 130.5 108.85) (end 130.5 83.2) (width 0.5) (layer "F.Cu") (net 13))
 (segment (start 170.95 80.1) (end 170.95 83.2) (width 0.5) (layer "F.Cu") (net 13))
 (segment (start 134.3 109.42) (end 131.07 109.42) (width 0.5) (layer "F.Cu") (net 13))
 (segment (start 135.2 78) (end 168.85 78) (width 0.5) (layer "F.Cu") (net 13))
 (segment (start 131.07 109.42) (end 130.5 108.85) (width 0.5) (layer "F.Cu") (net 13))
 (segment (start 130.5 83.2) (end 133.9 83.2) (width 0.5) (layer "F.Cu") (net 13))
 (segment (start 170.95 109.85) (end 170.95 83.2) (width 0.5) (layer "F.Cu") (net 13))
 (segment (start 135.2 83.2) (end 135.2 78) (width 0.5) (layer "F.Cu") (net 13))
 (segment (start 135.2 81.9) (end 135.2 81.25) (width 0.5) (layer "F.Cu") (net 13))
 (segment (start 170.95 109.85) (end 170.95 112.51) (width 0.5) (layer "F.Cu") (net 13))
 (segment (start 133.9 83.2) (end 134.55 83.2) (width 0.5) (layer "F.Cu") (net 13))
 (segment (start 135.2 82.55) (end 135.2 81.25) (width 0.5) (layer "F.Cu") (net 13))
 (segment (start 170.95 83.2) (end 170.95 81.9) (width 0.5) (layer "F.Cu") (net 13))
 (segment (start 168.85 78) (end 170.95 80.1) (width 0.5) (layer "F.Cu") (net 13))
 (segment (start 167.2 113.16) (end 170.3 113.16) (width 0.5) (layer "F.Cu") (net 13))
 (segment (start 133.9 83.2) (end 135.2 83.2) (width 0.5) (layer "F.Cu") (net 13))
 (segment (start 170.95 112.51) (end 170.3 113.16) (width 0.5) (layer "F.Cu") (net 13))
 (segment (start 167.2 115.7) (end 174.3 115.7) (width 0.5) (layer "F.Cu") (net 12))
 (segment (start 133.9 81.25) (end 129.35 81.25) (width 0.5) (layer "F.Cu") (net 12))
 (segment (start 133.9 76.7) (end 133.9 81.25) (width 0.5) (layer "F.Cu") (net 12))
 (segment (start 171.35 76.7) (end 133.9 76.7) (width 0.5) (layer "F.Cu") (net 12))
 (segment (start 129.35 111.8) (end 130 112.45) (width 0.5) (layer "F.Cu") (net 12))
 (segment (start 175.5 80.85) (end 171.35 76.7) (width 0.5) (layer "F.Cu") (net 12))
 (segment (start 175.5 114.5) (end 175.5 80.85) (width 0.5) (layer "F.Cu") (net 12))
 (segment (start 130 112.45) (end 133.81 112.45) (width 0.5) (layer "F.Cu") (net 12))
 (segment (start 129.35 81.25) (end 129.35 111.8) (width 0.5) (layer "F.Cu") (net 12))
 (segment (start 133.81 112.45) (end 134.3 111.96) (width 0.5) (layer "F.Cu") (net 12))
 (segment (start 167.4 115.9) (end 168.5 115.9) (width 0.5) (layer "F.Cu") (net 12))
 (segment (start 174.3 115.7) (end 175.5 114.5) (width 0.5) (layer "F.Cu") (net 12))
 (segment (start 177 82.55) (end 177 122) (width 0.5) (layer "F.Cu") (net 5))
 (segment (start 177 122) (end 175.68 123.32) (width 0.5) (layer "F.Cu") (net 5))
 (segment (start 177 82.55) (end 176.92 82.47) (width 0.5) (layer "F.Cu") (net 5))
 (segment (start 176.92 82.47) (end 176.92 75.695) (width 0.5) (layer "F.Cu") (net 5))
 (segment (start 175.68 123.32) (end 167.2 123.32) (width 0.5) (layer "F.Cu") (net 5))
 (segment (start 149.15 130) (end 147 127.85) (width 0.5) (layer "F.Cu") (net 26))
 (segment (start 147 115.8) (end 146.9 115.7) (width 0.5) (layer "F.Cu") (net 26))
 (segment (start 190 99.9) (end 190 122.35) (width 0.5) (layer "F.Cu") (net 26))
 (segment (start 188.65 98.55) (end 190 99.9) (width 0.5) (layer "F.Cu") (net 26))
 (segment (start 146.9 115.7) (end 151.96 115.7) (width 0.5) (layer "F.Cu") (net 26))
 (segment (start 147 127.85) (end 147 115.8) (width 0.5) (layer "F.Cu") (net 26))
 (segment (start 182.35 130) (end 149.15 130) (width 0.5) (layer "F.Cu") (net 26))
 (segment (start 190 122.35) (end 182.35 130) (width 0.5) (layer "F.Cu") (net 26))
 (segment (start 184.5 99) (end 184.95 98.55) (width 0.5) (layer "F.Cu") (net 26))
 (segment (start 184.95 98.55) (end 188.65 98.55) (width 0.5) (layer "F.Cu") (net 26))
 (segment (start 147.65 131.5) (end 145.5 129.35) (width 0.5) (layer "F.Cu") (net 27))
 (segment (start 191.1 123.75) (end 183.35 131.5) (width 0.5) (layer "F.Cu") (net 27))
 (segment (start 189.11 96.46) (end 191.1 98.45) (width 0.5) (layer "F.Cu") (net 27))
 (segment (start 145.66 113.16) (end 151.96 113.16) (width 0.5) (layer "F.Cu") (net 27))
 (segment (start 145.6 113.1) (end 145.66 113.16) (width 0.5) (layer "F.Cu") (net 27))
 (segment (start 145.5 129.35) (end 145.5 113.2) (width 0.5) (layer "F.Cu") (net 27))
 (segment (start 184.5 96.46) (end 189.11 96.46) (width 0.5) (layer "F.Cu") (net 27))
 (segment (start 183.35 131.5) (end 147.65 131.5) (width 0.5) (layer "F.Cu") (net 27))
 (segment (start 145.5 113.2) (end 145.6 113.1) (width 0.5) (layer "F.Cu") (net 27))
 (segment (start 191.1 98.45) (end 191.1 123.75) (width 0.5) (layer "F.Cu") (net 27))
 (segment (start 145.6 132.6) (end 145.6 132.45) (width 0.5) (layer "F.Cu") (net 28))
 (segment (start 190 93.92) (end 192.4 96.32) (width 0.5) (layer "F.Cu") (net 28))
 (segment (start 144 111.45) (end 144.83 110.62) (width 0.5) (layer "F.Cu") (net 28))
 (segment (start 184.5 93.92) (end 190 93.92) (width 0.5) (layer "F.Cu") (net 28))
 (segment (start 185.25 132.6) (end 145.6 132.6) (width 0.5) (layer "F.Cu") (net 28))
 (segment (start 192.4 96.32) (end 192.4 125.45) (width 0.5) (layer "F.Cu") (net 28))
 (segment (start 192.4 125.45) (end 185.25 132.6) (width 0.5) (layer "F.Cu") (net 28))
 (segment (start 144.83 110.62) (end 151.96 110.62) (width 0.5) (layer "F.Cu") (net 28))
 (segment (start 145.6 132.45) (end 144 130.85) (width 0.5) (layer "F.Cu") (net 28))
 (segment (start 144 130.85) (end 144 111.45) (width 0.5) (layer "F.Cu") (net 28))
 (segment (start 193.7 93.05) (end 193.7 126.65) (width 0.5) (layer "F.Cu") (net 29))
 (segment (start 184.5 91.38) (end 192.03 91.38) (width 0.5) (layer "F.Cu") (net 29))
 (segment (start 145.05 133.9) (end 142.5 131.35) (width 0.5) (layer "F.Cu") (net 29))
 (segment (start 193.7 126.65) (end 186.45 133.9) (width 0.5) (layer "F.Cu") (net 29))
 (segment (start 142.35 108.55) (end 142.82 108.08) (width 0.5) (layer "F.Cu") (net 29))
 (segment (start 192.03 91.38) (end 193.7 93.05) (width 0.5) (layer "F.Cu") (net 29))
 (segment (start 142.82 108.08) (end 151.96 108.08) (width 0.5) (layer "F.Cu") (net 29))
 (segment (start 186.45 133.9) (end 145.05 133.9) (width 0.5) (layer "F.Cu") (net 29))
 (segment (start 142.5 108.7) (end 142.35 108.55) (width 0.5) (layer "F.Cu") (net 29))
 (segment (start 142.5 131.35) (end 142.5 108.7) (width 0.5) (layer "F.Cu") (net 29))
 (segment (start 141 107.3) (end 141.95 106.35) (width 0.5) (layer "F.Cu") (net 30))
 (segment (start 141.95 106.35) (end 150 106.35) (width 0.5) (layer "F.Cu") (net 30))
 (segment (start 184.5 88.84) (end 193.51 88.84) (width 0.5) (layer "F.Cu") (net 30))
 (segment (start 141 132.4) (end 141 107.3) (width 0.5) (layer "F.Cu") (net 30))
 (segment (start 150.81 105.54) (end 151.96 105.54) (width 0.5) (layer "F.Cu") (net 30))
 (segment (start 195 90.33) (end 195 127.85) (width 0.5) (layer "F.Cu") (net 30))
 (segment (start 187.65 135.2) (end 143.8 135.2) (width 0.5) (layer "F.Cu") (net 30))
 (segment (start 150 106.35) (end 150.81 105.54) (width 0.5) (layer "F.Cu") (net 30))
 (segment (start 143.8 135.2) (end 141 132.4) (width 0.5) (layer "F.Cu") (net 30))
 (segment (start 195 127.85) (end 187.65 135.2) (width 0.5) (layer "F.Cu") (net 30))
 (segment (start 193.51 88.84) (end 195 90.33) (width 0.5) (layer "F.Cu") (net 30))
 (segment (start 195.65 79.455) (end 194.155 77.96) (width 0.5) (layer "F.Cu") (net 32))
 (segment (start 154.5 124.85) (end 158.15 128.5) (width 0.5) (layer "F.Cu") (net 32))
 (segment (start 154.5 103.35) (end 154.5 124.85) (width 0.5) (layer "F.Cu") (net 32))
 (segment (start 182.475 83.875) (end 182.5 83.85) (width 0.5) (layer "F.Cu") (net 32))
 (segment (start 188.5 103.85) (end 186.5 101.85) (width 0.5) (layer "F.Cu") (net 32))
 (segment (start 187.2 83.875) (end 187.2 86.7) (width 0.5) (layer "F.Cu") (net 32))
 (segment (start 183 101.85) (end 181.5 100.35) (width 0.5) (layer "F.Cu") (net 32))
 (segment (start 188.5 119.85) (end 188.5 103.85) (width 0.5) (layer "F.Cu") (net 32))
 (segment (start 181.5 100.35) (end 181.5 84.85) (width 0.5) (layer "F.Cu") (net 32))
 (segment (start 151.96 103) (end 154.15 103) (width 0.5) (layer "F.Cu") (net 32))
 (segment (start 154.15 103) (end 154.5 103.35) (width 0.5) (layer "F.Cu") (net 32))
 (segment (start 188 87.5) (end 194.6 87.5) (width 0.5) (layer "F.Cu") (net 32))
 (segment (start 181.5 84.85) (end 182.475 83.875) (width 0.5) (layer "F.Cu") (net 32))
 (segment (start 186.5 101.85) (end 183 101.85) (width 0.5) (layer "F.Cu") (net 32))
 (segment (start 194.6 87.5) (end 195.65 86.45) (width 0.5) (layer "F.Cu") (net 32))
 (segment (start 158.15 128.5) (end 179.85 128.5) (width 0.5) (layer "F.Cu") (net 32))
 (segment (start 182.475 83.875) (end 187.2 83.875) (width 0.5) (layer "F.Cu") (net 32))
 (segment (start 187.2 86.7) (end 188 87.5) (width 0.5) (layer "F.Cu") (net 32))
 (segment (start 195.65 86.45) (end 195.65 79.455) (width 0.5) (layer "F.Cu") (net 32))
 (segment (start 179.85 128.5) (end 188.5 119.85) (width 0.5) (layer "F.Cu") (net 32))
 (segment (start 179.46 79.655) (end 179.46 73.45) (width 0.5) (layer "F.Cu") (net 4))
 (segment (start 178.825 111.675) (end 179 111.85) (width 0.5) (layer "F.Cu") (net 4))
 (segment (start 184.35 111.85) (end 184.5 111.7) (width 0.5) (layer "F.Cu") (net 4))
 (segment (start 178.5 80.615) (end 179.46 79.655) (width 0.5) (layer "F.Cu") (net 4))
 (segment (start 172.9 73.45) (end 179.46 73.45) (width 0.5) (layer "F.Cu") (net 4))
 (segment (start 164.5 110.9) (end 164.5 125.5) (width 0.5) (layer "F.Cu") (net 4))
 (segment (start 164.5 125.5) (end 178 125.5) (width 0.5) (layer "F.Cu") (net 4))
 (segment (start 190.845 75.42) (end 190.845 74.495) (width 0.5) (layer "F.Cu") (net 4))
 (segment (start 178.5 110.5) (end 178.5 80.615) (width 0.5) (layer "F.Cu") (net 4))
 (segment (start 180.5 111.85) (end 184.35 111.85) (width 0.5) (layer "F.Cu") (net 4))
 (segment (start 178.5 109.9) (end 178.5 111.35) (width 0.5) (layer "F.Cu") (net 4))
 (segment (start 155.41 87.76) (end 157.5 89.85) (width 0.5) (layer "F.Cu") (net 4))
 (segment (start 179.46 73.45) (end 189.8 73.45) (width 0.5) (layer "F.Cu") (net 4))
 (segment (start 151.96 87.76) (end 155.41 87.76) (width 0.5) (layer "F.Cu") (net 4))
 (segment (start 163 74.1) (end 172.25 74.1) (width 0.5) (layer "F.Cu") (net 4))
 (segment (start 157.5 103.9) (end 164.5 110.9) (width 0.5) (layer "F.Cu") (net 4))
 (segment (start 180 123.5) (end 180 111.85) (width 0.5) (layer "F.Cu") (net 4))
 (segment (start 178.46 111.31) (end 178.825 111.675) (width 0.5) (layer "F.Cu") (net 4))
 (segment (start 190.845 74.495) (end 189.8 73.45) (width 0.5) (layer "F.Cu") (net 4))
 (segment (start 180.5 111.85) (end 179 111.85) (width 0.5) (layer "F.Cu") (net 4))
 (segment (start 178.5 109.9) (end 178.5 110.5) (width 0.5) (layer "F.Cu") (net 4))
 (segment (start 157.5 89.85) (end 157.5 103.9) (width 0.5) (layer "F.Cu") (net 4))
 (segment (start 178.5 111.35) (end 178.825 111.675) (width 0.5) (layer "F.Cu") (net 4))
 (segment (start 178 125.5) (end 180 123.5) (width 0.5) (layer "F.Cu") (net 4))
 (segment (start 179.5 111.85) (end 180.5 111.85) (width 0.5) (layer "F.Cu") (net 4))
 (segment (start 178.5 110.5) (end 178.5 110.85) (width 0.5) (layer "F.Cu") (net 4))
 (segment (start 172.25 74.1) (end 172.9 73.45) (width 0.5) (layer "F.Cu") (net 4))
 (segment (start 166.4 68.25) (end 166.105 67.955) (width 0.5) (layer "F.Cu") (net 1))
 (segment (start 176.8 69.55) (end 186.7 69.55) (width 0.5) (layer "F.Cu") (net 1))
 (segment (start 169.65 71.75) (end 174.6 71.75) (width 0.5) (layer "F.Cu") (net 1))
 (segment (start 166.4 68.25) (end 166.4 71.5) (width 0.5) (layer "F.Cu") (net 1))
 (segment (start 166.4 71.5) (end 166.65 71.75) (width 0.5) (layer "F.Cu") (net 1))
 (segment (start 174.6 71.75) (end 176.8 69.55) (width 0.5) (layer "F.Cu") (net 1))
 (segment (start 166.105 67.955) (end 161.79 67.955) (width 0.5) (layer "F.Cu") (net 1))
 (segment (start 166.65 71.75) (end 169.65 71.75) (width 0.5) (layer "F.Cu") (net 1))
 (segment (start 154.3 74.1) (end 158.6 74.1) (width 0.5) (layer "F.Cu") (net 3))
 (segment (start 157.36 69.255) (end 154.595 69.255) (width 0.5) (layer "F.Cu") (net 3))
 (segment (start 154.3 69.55) (end 154.3 74.1) (width 0.5) (layer "F.Cu") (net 3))
 (segment (start 154.595 69.255) (end 154.3 69.55) (width 0.5) (layer "F.Cu") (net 3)))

